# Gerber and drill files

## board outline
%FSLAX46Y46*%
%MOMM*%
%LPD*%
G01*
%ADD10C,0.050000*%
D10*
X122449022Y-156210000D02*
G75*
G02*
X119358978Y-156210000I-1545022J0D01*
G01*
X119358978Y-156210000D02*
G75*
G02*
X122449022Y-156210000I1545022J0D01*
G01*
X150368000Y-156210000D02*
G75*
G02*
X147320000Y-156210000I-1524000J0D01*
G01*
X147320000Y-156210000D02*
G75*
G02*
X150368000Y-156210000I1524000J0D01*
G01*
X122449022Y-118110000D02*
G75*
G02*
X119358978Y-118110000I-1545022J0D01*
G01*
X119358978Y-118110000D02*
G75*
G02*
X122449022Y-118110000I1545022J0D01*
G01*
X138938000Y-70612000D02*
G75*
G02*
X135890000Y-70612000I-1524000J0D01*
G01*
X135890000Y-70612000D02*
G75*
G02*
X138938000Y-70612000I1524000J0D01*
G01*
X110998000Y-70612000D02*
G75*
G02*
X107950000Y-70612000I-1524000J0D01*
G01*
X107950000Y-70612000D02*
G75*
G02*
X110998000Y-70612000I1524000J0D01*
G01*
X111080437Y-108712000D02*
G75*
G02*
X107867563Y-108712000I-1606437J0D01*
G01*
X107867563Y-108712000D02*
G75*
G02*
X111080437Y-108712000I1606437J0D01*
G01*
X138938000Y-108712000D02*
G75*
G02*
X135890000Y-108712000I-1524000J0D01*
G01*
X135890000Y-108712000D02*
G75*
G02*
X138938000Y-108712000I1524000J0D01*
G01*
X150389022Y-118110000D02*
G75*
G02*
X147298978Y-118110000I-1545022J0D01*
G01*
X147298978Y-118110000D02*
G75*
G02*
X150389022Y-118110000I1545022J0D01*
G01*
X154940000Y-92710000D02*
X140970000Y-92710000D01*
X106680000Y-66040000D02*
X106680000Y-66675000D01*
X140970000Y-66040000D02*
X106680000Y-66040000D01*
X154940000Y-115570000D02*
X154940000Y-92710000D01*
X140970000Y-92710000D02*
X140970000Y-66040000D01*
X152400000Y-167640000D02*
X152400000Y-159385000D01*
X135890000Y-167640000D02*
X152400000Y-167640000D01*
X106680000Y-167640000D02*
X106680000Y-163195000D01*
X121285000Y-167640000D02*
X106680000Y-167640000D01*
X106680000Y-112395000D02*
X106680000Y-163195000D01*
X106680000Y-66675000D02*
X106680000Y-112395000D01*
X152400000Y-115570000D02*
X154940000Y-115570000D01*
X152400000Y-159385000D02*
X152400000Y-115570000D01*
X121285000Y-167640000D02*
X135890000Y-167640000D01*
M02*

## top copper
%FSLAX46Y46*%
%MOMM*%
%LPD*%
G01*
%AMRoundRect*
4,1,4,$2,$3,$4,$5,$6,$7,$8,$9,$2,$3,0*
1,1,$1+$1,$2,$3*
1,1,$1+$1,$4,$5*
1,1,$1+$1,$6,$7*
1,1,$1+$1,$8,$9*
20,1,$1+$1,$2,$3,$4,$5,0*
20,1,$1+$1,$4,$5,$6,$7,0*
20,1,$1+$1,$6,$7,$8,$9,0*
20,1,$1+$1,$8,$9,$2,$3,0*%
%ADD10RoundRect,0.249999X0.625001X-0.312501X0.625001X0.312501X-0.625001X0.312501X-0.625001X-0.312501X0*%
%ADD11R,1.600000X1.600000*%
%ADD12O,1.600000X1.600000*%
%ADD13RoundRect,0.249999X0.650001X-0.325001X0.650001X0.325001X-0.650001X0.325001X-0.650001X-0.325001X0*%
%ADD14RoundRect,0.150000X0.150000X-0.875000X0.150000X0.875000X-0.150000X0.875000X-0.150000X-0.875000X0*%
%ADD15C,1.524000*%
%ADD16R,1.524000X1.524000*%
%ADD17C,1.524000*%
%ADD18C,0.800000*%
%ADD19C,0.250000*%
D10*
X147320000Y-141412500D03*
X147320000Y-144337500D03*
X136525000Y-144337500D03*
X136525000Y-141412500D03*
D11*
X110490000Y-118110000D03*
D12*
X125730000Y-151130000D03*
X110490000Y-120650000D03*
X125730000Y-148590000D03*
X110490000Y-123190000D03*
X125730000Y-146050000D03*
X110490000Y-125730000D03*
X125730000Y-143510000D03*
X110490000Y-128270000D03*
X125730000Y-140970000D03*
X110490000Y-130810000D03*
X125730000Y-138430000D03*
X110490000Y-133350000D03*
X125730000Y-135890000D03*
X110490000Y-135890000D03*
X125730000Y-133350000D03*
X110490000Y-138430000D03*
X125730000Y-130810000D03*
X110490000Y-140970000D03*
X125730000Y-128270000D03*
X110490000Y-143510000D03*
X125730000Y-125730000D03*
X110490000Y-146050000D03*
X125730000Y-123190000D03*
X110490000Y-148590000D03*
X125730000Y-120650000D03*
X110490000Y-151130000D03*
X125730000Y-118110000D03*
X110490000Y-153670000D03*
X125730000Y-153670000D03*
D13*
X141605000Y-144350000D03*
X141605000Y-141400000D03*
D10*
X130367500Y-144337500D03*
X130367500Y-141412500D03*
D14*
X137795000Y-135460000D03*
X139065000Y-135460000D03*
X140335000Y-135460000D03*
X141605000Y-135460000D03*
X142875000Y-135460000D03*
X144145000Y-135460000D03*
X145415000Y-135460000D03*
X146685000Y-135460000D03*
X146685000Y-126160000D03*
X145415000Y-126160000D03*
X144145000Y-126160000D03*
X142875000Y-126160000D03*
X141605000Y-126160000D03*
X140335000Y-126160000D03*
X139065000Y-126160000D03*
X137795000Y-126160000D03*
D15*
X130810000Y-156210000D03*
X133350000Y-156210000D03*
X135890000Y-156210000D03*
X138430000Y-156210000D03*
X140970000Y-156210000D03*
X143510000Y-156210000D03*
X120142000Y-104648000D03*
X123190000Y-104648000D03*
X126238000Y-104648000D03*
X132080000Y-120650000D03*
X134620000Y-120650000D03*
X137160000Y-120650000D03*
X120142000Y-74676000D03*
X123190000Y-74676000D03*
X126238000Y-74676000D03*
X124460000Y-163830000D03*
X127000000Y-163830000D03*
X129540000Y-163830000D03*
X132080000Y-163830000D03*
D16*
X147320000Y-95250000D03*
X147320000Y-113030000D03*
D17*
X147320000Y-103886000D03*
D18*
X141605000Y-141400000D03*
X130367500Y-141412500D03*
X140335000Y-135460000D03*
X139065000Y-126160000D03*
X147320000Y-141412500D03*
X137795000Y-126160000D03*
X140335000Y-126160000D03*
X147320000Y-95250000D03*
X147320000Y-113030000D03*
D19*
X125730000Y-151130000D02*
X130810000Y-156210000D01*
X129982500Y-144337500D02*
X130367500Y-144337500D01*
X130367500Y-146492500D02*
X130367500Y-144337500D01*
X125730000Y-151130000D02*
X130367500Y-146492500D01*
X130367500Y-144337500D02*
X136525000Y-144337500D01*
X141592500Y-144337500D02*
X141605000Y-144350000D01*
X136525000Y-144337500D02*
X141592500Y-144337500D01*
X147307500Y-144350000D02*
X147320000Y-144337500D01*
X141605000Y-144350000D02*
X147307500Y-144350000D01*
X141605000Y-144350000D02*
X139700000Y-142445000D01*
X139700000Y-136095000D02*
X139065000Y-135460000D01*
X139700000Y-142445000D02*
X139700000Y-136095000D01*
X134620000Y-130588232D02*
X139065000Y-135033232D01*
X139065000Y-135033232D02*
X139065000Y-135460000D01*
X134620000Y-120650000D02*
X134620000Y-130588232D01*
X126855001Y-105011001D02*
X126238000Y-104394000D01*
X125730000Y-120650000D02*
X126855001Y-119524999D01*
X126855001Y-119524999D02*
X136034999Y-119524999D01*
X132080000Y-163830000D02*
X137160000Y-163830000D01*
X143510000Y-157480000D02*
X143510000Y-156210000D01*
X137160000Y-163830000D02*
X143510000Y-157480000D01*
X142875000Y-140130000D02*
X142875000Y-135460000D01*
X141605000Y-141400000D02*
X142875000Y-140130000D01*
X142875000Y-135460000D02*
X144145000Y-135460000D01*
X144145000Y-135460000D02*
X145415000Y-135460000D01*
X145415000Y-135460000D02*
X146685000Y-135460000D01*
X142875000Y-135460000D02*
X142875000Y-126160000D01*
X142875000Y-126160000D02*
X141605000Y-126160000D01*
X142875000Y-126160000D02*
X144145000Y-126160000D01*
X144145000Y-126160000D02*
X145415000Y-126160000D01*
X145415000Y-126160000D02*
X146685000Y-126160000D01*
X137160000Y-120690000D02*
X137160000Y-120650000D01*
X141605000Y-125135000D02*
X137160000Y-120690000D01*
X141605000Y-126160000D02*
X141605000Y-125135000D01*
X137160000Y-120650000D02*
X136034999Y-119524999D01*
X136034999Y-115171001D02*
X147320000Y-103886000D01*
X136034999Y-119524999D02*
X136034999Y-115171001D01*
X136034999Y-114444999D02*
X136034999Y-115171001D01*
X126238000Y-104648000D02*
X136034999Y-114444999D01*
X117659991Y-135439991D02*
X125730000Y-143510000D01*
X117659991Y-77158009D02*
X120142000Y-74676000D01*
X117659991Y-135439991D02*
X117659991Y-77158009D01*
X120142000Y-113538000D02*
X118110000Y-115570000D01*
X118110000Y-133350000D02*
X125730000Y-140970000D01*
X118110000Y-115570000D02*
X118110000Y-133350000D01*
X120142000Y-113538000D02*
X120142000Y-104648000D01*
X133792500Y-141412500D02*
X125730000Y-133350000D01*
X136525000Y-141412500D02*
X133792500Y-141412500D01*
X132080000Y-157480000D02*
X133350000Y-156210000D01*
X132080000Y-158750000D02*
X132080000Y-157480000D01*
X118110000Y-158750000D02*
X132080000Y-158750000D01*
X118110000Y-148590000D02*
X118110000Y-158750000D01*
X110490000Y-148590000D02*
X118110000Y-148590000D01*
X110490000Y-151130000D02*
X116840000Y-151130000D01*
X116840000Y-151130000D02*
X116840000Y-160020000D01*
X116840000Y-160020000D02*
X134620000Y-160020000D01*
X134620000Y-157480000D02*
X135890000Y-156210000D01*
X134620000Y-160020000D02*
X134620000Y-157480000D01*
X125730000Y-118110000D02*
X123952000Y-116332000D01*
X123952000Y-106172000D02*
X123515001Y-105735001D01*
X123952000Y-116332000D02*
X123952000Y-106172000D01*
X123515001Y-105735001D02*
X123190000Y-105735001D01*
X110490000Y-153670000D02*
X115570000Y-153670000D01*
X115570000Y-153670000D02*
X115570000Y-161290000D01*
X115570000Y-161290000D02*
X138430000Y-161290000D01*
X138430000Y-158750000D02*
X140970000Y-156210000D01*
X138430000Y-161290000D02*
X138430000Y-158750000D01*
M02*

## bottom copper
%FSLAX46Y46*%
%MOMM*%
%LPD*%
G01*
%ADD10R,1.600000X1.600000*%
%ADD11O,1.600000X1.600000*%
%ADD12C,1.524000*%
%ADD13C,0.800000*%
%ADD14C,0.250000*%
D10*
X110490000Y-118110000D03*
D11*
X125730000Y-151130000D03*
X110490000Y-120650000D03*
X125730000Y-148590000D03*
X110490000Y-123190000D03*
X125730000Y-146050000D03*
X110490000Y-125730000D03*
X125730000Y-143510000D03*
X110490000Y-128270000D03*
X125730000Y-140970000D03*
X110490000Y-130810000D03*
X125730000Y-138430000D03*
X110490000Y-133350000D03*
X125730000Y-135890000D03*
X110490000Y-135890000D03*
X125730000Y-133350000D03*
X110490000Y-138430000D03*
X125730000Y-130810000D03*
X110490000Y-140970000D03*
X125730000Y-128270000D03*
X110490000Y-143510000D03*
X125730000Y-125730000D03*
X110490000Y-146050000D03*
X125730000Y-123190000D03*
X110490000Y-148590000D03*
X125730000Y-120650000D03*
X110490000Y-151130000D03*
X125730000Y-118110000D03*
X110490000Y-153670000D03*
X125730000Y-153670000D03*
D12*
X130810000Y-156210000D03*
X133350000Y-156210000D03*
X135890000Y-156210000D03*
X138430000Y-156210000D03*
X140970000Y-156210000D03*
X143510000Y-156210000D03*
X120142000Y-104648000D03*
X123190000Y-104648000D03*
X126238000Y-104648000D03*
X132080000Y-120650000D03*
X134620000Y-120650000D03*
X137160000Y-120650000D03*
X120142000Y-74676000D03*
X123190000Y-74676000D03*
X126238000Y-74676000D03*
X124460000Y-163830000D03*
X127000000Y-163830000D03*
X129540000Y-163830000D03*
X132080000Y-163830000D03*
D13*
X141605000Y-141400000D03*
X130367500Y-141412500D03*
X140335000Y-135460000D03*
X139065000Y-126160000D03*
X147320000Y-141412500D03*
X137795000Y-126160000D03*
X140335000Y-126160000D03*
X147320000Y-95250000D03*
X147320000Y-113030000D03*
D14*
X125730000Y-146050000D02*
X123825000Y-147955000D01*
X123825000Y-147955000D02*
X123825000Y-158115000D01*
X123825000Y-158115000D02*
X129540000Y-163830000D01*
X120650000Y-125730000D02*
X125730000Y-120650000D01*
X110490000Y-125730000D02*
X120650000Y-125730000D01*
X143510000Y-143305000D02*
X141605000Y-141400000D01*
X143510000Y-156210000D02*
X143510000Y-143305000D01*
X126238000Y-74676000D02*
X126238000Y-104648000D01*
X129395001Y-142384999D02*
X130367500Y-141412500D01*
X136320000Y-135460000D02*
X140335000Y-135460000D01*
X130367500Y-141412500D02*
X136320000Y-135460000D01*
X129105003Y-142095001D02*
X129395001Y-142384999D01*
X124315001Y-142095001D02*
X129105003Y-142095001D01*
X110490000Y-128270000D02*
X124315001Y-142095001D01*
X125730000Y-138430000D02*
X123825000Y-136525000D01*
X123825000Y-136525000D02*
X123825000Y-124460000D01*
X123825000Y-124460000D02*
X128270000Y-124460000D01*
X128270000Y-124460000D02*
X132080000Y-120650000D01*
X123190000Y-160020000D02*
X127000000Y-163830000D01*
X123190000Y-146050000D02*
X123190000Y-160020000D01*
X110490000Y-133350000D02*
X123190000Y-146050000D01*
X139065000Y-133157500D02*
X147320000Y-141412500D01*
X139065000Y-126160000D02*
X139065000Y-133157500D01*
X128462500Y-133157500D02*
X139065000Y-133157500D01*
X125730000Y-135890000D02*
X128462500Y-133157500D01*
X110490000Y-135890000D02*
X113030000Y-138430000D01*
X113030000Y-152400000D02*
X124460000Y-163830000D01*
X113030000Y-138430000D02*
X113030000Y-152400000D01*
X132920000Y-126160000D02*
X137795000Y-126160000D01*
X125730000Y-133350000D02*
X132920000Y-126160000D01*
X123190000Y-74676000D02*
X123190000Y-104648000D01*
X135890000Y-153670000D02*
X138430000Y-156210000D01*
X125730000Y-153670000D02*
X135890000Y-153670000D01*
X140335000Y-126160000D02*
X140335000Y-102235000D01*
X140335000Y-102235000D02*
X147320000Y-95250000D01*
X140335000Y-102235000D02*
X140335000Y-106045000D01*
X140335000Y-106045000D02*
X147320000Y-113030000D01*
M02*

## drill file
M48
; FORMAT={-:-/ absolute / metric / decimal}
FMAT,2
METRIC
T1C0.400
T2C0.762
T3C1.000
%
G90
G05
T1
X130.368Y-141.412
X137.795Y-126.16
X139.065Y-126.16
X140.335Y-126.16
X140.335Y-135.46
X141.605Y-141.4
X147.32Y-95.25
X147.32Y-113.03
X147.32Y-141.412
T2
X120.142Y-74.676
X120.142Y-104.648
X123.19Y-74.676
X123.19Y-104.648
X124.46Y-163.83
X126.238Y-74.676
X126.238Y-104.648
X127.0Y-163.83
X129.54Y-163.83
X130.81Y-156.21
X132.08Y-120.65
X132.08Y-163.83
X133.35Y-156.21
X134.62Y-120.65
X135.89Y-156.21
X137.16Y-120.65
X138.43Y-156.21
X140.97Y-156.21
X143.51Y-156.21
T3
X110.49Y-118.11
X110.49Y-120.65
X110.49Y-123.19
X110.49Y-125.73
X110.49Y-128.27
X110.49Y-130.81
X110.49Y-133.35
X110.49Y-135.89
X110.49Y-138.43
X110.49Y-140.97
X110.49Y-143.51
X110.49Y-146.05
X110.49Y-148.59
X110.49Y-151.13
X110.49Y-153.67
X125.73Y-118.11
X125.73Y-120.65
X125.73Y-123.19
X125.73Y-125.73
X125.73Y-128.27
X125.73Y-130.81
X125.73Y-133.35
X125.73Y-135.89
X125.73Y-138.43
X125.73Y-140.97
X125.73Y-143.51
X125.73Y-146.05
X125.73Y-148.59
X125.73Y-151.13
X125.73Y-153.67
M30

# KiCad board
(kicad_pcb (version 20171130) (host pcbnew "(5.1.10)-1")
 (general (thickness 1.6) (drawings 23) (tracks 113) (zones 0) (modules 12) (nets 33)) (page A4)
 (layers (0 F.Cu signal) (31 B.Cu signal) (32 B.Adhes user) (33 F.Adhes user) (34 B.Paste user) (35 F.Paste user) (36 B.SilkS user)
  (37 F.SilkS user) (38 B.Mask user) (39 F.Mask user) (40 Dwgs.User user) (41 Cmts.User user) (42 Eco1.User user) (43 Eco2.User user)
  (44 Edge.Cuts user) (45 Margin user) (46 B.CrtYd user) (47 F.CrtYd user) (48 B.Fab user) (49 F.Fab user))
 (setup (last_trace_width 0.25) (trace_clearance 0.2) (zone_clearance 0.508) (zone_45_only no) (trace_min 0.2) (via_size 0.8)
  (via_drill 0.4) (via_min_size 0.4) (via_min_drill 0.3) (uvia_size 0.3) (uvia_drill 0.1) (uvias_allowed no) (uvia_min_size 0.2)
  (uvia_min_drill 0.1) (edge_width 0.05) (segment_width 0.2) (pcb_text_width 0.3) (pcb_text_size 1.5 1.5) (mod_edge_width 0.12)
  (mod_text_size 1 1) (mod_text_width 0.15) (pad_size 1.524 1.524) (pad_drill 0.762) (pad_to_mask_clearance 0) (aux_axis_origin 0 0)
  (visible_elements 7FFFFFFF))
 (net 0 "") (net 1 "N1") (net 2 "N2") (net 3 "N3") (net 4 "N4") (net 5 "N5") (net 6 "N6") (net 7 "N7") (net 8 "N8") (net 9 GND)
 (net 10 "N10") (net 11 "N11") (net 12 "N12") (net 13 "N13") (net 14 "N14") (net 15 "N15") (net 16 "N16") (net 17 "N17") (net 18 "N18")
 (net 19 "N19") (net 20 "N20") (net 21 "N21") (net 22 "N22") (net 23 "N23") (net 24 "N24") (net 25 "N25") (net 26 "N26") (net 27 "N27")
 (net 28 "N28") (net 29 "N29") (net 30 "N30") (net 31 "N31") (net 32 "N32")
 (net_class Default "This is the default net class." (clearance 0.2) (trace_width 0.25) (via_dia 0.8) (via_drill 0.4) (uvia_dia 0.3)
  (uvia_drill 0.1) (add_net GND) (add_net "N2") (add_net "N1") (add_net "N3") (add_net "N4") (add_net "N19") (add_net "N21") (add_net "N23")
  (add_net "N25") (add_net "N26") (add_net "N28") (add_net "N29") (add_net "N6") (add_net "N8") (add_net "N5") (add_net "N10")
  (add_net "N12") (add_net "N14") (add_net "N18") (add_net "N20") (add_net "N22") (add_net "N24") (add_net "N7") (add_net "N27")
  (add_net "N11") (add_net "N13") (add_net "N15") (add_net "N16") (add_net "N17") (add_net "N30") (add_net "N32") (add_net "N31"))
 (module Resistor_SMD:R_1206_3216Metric (layer F.Cu) (at 147.32 142.875 90)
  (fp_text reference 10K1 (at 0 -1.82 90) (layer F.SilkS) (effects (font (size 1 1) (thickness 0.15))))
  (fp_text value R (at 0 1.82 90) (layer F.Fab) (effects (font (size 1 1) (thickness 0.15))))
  (pad 2 smd roundrect (at 1.4625 0 90) (size 1.125 1.75) (layers F.Cu F.Paste F.Mask) (roundrect_rratio 0.2222213333333333) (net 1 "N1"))
  (pad 1 smd roundrect (at -1.4625 0 90) (size 1.125 1.75) (layers F.Cu F.Paste F.Mask) (roundrect_rratio 0.2222213333333333) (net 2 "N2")))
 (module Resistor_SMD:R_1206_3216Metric (layer F.Cu) (at 136.525 142.875 90)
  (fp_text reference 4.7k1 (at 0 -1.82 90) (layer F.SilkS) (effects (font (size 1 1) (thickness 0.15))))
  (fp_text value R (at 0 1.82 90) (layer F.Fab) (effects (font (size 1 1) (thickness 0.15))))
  (pad 1 smd roundrect (at -1.4625 0 90) (size 1.125 1.75) (layers F.Cu F.Paste F.Mask) (roundrect_rratio 0.2222213333333333) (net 2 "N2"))
  (pad 2 smd roundrect (at 1.4625 0 90) (size 1.125 1.75) (layers F.Cu F.Paste F.Mask) (roundrect_rratio 0.2222213333333333) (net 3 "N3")))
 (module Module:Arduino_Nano (layer F.Cu) (at 110.49 118.11)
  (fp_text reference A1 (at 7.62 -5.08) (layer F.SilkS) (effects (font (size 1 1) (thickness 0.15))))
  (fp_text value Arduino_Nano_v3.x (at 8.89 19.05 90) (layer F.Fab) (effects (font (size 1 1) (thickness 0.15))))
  (pad 1 thru_hole rect (at 0 0) (size 1.6 1.6) (drill 1) (layers *.Cu *.Mask) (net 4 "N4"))
  (pad 17 thru_hole oval (at 15.24 33.02) (size 1.6 1.6) (drill 1) (layers *.Cu *.Mask) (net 2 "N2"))
  (pad 2 thru_hole oval (at 0 2.54) (size 1.6 1.6) (drill 1) (layers *.Cu *.Mask) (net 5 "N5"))
  (pad 18 thru_hole oval (at 15.24 30.48) (size 1.6 1.6) (drill 1) (layers *.Cu *.Mask) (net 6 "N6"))
  (pad 3 thru_hole oval (at 0 5.08) (size 1.6 1.6) (drill 1) (layers *.Cu *.Mask) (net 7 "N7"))
  (pad 19 thru_hole oval (at 15.24 27.94) (size 1.6 1.6) (drill 1) (layers *.Cu *.Mask) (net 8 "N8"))
  (pad 4 thru_hole oval (at 0 7.62) (size 1.6 1.6) (drill 1) (layers *.Cu *.Mask) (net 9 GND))
  (pad 20 thru_hole oval (at 15.24 25.4) (size 1.6 1.6) (drill 1) (layers *.Cu *.Mask) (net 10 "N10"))
  (pad 5 thru_hole oval (at 0 10.16) (size 1.6 1.6) (drill 1) (layers *.Cu *.Mask) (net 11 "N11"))
  (pad 21 thru_hole oval (at 15.24 22.86) (size 1.6 1.6) (drill 1) (layers *.Cu *.Mask) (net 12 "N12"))
  (pad 6 thru_hole oval (at 0 12.7) (size 1.6 1.6) (drill 1) (layers *.Cu *.Mask) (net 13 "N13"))
  (pad 22 thru_hole oval (at 15.24 20.32) (size 1.6 1.6) (drill 1) (layers *.Cu *.Mask) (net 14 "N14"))
  (pad 7 thru_hole oval (at 0 15.24) (size 1.6 1.6) (drill 1) (layers *.Cu *.Mask) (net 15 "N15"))
  (pad 23 thru_hole oval (at 15.24 17.78) (size 1.6 1.6) (drill 1) (layers *.Cu *.Mask) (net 1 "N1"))
  (pad 8 thru_hole oval (at 0 17.78) (size 1.6 1.6) (drill 1) (layers *.Cu *.Mask) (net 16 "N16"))
  (pad 24 thru_hole oval (at 15.24 15.24) (size 1.6 1.6) (drill 1) (layers *.Cu *.Mask) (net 3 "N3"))
  (pad 9 thru_hole oval (at 0 20.32) (size 1.6 1.6) (drill 1) (layers *.Cu *.Mask) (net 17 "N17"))
  (pad 25 thru_hole oval (at 15.24 12.7) (size 1.6 1.6) (drill 1) (layers *.Cu *.Mask) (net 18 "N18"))
  (pad 10 thru_hole oval (at 0 22.86) (size 1.6 1.6) (drill 1) (layers *.Cu *.Mask) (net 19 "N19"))
  (pad 26 thru_hole oval (at 15.24 10.16) (size 1.6 1.6) (drill 1) (layers *.Cu *.Mask) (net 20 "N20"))
  (pad 11 thru_hole oval (at 0 25.4) (size 1.6 1.6) (drill 1) (layers *.Cu *.Mask) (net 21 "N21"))
  (pad 27 thru_hole oval (at 15.24 7.62) (size 1.6 1.6) (drill 1) (layers *.Cu *.Mask) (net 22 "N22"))
  (pad 12 thru_hole oval (at 0 27.94) (size 1.6 1.6) (drill 1) (layers *.Cu *.Mask) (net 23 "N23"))
  (pad 28 thru_hole oval (at 15.24 5.08) (size 1.6 1.6) (drill 1) (layers *.Cu *.Mask) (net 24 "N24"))
  (pad 13 thru_hole oval (at 0 30.48) (size 1.6 1.6) (drill 1) (layers *.Cu *.Mask) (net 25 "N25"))
  (pad 29 thru_hole oval (at 15.24 2.54) (size 1.6 1.6) (drill 1) (layers *.Cu *.Mask) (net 9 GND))
  (pad 14 thru_hole oval (at 0 33.02) (size 1.6 1.6) (drill 1) (layers *.Cu *.Mask) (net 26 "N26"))
  (pad 30 thru_hole oval (at 15.24 0) (size 1.6 1.6) (drill 1) (layers *.Cu *.Mask) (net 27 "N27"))
  (pad 15 thru_hole oval (at 0 35.56) (size 1.6 1.6) (drill 1) (layers *.Cu *.Mask) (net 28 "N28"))
  (pad 16 thru_hole oval (at 15.24 35.56) (size 1.6 1.6) (drill 1) (layers *.Cu *.Mask) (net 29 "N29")))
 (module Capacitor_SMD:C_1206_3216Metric (layer F.Cu) (at 141.605 142.875 90)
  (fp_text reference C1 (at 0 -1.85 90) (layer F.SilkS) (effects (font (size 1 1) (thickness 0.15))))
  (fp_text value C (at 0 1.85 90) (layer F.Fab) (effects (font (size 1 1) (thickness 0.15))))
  (pad 1 smd roundrect (at -1.475 0 90) (size 1.15 1.8) (layers F.Cu F.Paste F.Mask) (roundrect_rratio 0.2173904347826087) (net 2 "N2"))
  (pad 2 smd roundrect (at 1.475 0 90) (size 1.15 1.8) (layers F.Cu F.Paste F.Mask) (roundrect_rratio 0.2173904347826087) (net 9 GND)))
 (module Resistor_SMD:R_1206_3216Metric (layer F.Cu) (at 130.3675 142.875 90)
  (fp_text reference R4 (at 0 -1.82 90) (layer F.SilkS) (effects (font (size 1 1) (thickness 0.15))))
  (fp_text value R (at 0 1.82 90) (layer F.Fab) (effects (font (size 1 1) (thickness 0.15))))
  (pad 1 smd roundrect (at -1.4625 0 90) (size 1.125 1.75) (layers F.Cu F.Paste F.Mask) (roundrect_rratio 0.2222213333333333) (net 2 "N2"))
  (pad 2 smd roundrect (at 1.4625 0 90) (size 1.125 1.75) (layers F.Cu F.Paste F.Mask) (roundrect_rratio 0.2222213333333333) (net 11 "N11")))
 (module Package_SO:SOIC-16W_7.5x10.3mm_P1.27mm (layer F.Cu) (at 142.24 130.81 90)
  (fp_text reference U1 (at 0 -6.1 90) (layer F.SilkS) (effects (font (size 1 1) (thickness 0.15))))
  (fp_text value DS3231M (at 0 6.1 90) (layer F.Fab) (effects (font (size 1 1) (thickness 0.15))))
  (pad 1 smd roundrect (at -4.65 -4.445 90) (size 2.05 0.6) (layers F.Cu F.Paste F.Mask) (roundrect_rratio 0.25) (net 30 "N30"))
  (pad 2 smd roundrect (at -4.65 -3.175 90) (size 2.05 0.6) (layers F.Cu F.Paste F.Mask) (roundrect_rratio 0.25) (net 2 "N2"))
  (pad 3 smd roundrect (at -4.65 -1.905 90) (size 2.05 0.6) (layers F.Cu F.Paste F.Mask) (roundrect_rratio 0.25) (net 11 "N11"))
  (pad 4 smd roundrect (at -4.65 -0.635 90) (size 2.05 0.6) (layers F.Cu F.Paste F.Mask) (roundrect_rratio 0.25) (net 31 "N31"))
  (pad 5 smd roundrect (at -4.65 0.635 90) (size 2.05 0.6) (layers F.Cu F.Paste F.Mask) (roundrect_rratio 0.25) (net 9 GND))
  (pad 6 smd roundrect (at -4.65 1.905 90) (size 2.05 0.6) (layers F.Cu F.Paste F.Mask) (roundrect_rratio 0.25) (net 9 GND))
  (pad 7 smd roundrect (at -4.65 3.175 90) (size 2.05 0.6) (layers F.Cu F.Paste F.Mask) (roundrect_rratio 0.25) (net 9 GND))
  (pad 8 smd roundrect (at -4.65 4.445 90) (size 2.05 0.6) (layers F.Cu F.Paste F.Mask) (roundrect_rratio 0.25) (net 9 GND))
  (pad 9 smd roundrect (at 4.65 4.445 90) (size 2.05 0.6) (layers F.Cu F.Paste F.Mask) (roundrect_rratio 0.25) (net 9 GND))
  (pad 10 smd roundrect (at 4.65 3.175 90) (size 2.05 0.6) (layers F.Cu F.Paste F.Mask) (roundrect_rratio 0.25) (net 9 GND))
  (pad 11 smd roundrect (at 4.65 1.905 90) (size 2.05 0.6) (layers F.Cu F.Paste F.Mask) (roundrect_rratio 0.25) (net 9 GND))
  (pad 12 smd roundrect (at 4.65 0.635 90) (size 2.05 0.6) (layers F.Cu F.Paste F.Mask) (roundrect_rratio 0.25) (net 9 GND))
  (pad 13 smd roundrect (at 4.65 -0.635 90) (size 2.05 0.6) (layers F.Cu F.Paste F.Mask) (roundrect_rratio 0.25) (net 9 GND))
  (pad 14 smd roundrect (at 4.65 -1.905 90) (size 2.05 0.6) (layers F.Cu F.Paste F.Mask) (roundrect_rratio 0.25) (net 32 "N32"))
  (pad 15 smd roundrect (at 4.65 -3.175 90) (size 2.05 0.6) (layers F.Cu F.Paste F.Mask) (roundrect_rratio 0.25) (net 1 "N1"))
  (pad 16 smd roundrect (at 4.65 -4.445 90) (size 2.05 0.6) (layers F.Cu F.Paste F.Mask) (roundrect_rratio 0.25) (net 3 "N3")))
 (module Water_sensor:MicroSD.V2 (layer F.Cu) (at 138.43 153.67)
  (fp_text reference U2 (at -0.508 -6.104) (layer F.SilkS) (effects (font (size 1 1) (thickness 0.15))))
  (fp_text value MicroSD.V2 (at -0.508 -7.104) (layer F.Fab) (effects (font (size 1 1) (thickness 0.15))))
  (pad 1 thru_hole circle (at -7.62 2.54) (size 1.524 1.524) (drill 0.762) (layers *.Cu *.Mask) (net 2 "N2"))
  (pad 2 thru_hole circle (at -5.08 2.54) (size 1.524 1.524) (drill 0.762) (layers *.Cu *.Mask) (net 25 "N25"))
  (pad 3 thru_hole circle (at -2.54 2.54) (size 1.524 1.524) (drill 0.762) (layers *.Cu *.Mask) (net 26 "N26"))
  (pad 4 thru_hole circle (at 0 2.54) (size 1.524 1.524) (drill 0.762) (layers *.Cu *.Mask) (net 29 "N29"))
  (pad 5 thru_hole circle (at 2.54 2.54) (size 1.524 1.524) (drill 0.762) (layers *.Cu *.Mask) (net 28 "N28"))
  (pad 6 thru_hole circle (at 5.08 2.54) (size 1.524 1.524) (drill 0.762) (layers *.Cu *.Mask) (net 9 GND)))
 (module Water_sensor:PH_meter (layer F.Cu) (at 123.19 105.664)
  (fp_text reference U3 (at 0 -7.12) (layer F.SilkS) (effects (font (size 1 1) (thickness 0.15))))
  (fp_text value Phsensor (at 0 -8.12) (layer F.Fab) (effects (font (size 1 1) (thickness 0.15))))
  (pad 1 thru_hole circle (at -3.048 -1.016) (size 1.524 1.524) (drill 0.762) (layers *.Cu *.Mask) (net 12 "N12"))
  (pad 2 thru_hole circle (at 0 -1.016) (size 1.524 1.524) (drill 0.762) (layers *.Cu *.Mask) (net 22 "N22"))
  (pad 3 thru_hole circle (at 3.048 -1.016) (size 1.524 1.524) (drill 0.762) (layers *.Cu *.Mask) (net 9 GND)))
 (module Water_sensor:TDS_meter (layer B.Cu) (at 134.62 123.19)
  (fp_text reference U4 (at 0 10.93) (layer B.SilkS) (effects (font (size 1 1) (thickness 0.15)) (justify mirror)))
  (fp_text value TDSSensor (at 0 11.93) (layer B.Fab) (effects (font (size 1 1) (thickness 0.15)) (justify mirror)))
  (pad 1 thru_hole circle (at -2.54 -2.54) (size 1.524 1.524) (drill 0.762) (layers *.Cu *.Mask) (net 14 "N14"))
  (pad 2 thru_hole circle (at 0 -2.54) (size 1.524 1.524) (drill 0.762) (layers *.Cu *.Mask) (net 2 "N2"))
  (pad 3 thru_hole circle (at 2.54 -2.54) (size 1.524 1.524) (drill 0.762) (layers *.Cu *.Mask) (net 9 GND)))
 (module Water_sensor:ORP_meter (layer B.Cu) (at 123.19 73.66)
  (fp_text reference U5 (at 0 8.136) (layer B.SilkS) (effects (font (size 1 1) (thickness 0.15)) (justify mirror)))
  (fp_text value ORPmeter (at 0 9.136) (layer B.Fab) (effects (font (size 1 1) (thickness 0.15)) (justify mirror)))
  (pad 1 thru_hole circle (at -3.048 1.016) (size 1.524 1.524) (drill 0.762) (layers *.Cu *.Mask F.SilkS) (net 10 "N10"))
  (pad 2 thru_hole circle (at 0 1.016) (size 1.524 1.524) (drill 0.762) (layers *.Cu *.Mask F.SilkS) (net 22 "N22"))
  (pad 3 thru_hole circle (at 3.048 1.016) (size 1.524 1.524) (drill 0.762) (layers *.Cu *.Mask F.SilkS) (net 9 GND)))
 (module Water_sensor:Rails (layer F.Cu) (at 128.27 161.29)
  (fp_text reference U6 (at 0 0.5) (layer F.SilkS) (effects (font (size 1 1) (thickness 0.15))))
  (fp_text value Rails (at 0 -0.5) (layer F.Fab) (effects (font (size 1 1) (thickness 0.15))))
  (pad 1 thru_hole circle (at -3.81 2.54) (size 1.524 1.524) (drill 0.762) (layers *.Cu *.Mask) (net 16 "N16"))
  (pad 2 thru_hole circle (at -1.27 2.54) (size 1.524 1.524) (drill 0.762) (layers *.Cu *.Mask) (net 15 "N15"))
  (pad 3 thru_hole circle (at 1.27 2.54) (size 1.524 1.524) (drill 0.762) (layers *.Cu *.Mask) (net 8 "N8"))
  (pad 4 thru_hole circle (at 3.81 2.54) (size 1.524 1.524) (drill 0.762) (layers *.Cu *.Mask) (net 9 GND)))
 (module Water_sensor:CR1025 (layer F.Cu) (at 147.32 110.49)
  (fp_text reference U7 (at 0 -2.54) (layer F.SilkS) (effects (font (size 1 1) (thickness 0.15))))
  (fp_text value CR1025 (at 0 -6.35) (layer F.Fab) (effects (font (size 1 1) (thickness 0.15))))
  (pad 1 smd rect (at 0 -15.24) (size 1.524 1.524) (layers F.Cu F.Paste F.Mask) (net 32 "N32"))
  (pad 2 smd rect (at 0 2.54) (size 1.524 1.524) (layers F.Cu F.Paste F.Mask) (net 32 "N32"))
  (pad 3 smd circle (at 0 -6.604) (size 1.524 1.524) (layers F.Cu F.Paste F.Mask) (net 9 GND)))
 (gr_circle (center 120.904 156.21) (end 121.158 154.686) (layer Edge.Cuts) (width 0.05))
 (gr_circle (center 148.844 156.21) (end 148.844 157.734) (layer Edge.Cuts) (width 0.05))
 (gr_circle (center 120.904 118.11) (end 120.65 116.586) (layer Edge.Cuts) (width 0.05))
 (gr_circle (center 137.414 70.612) (end 137.414 69.088) (layer Edge.Cuts) (width 0.05))
 (gr_circle (center 109.474 70.612) (end 109.474 69.088) (layer Edge.Cuts) (width 0.05))
 (gr_circle (center 109.474 108.712) (end 109.982 107.188) (layer Edge.Cuts) (width 0.05))
 (gr_circle (center 137.414 108.712) (end 137.414 107.188) (layer Edge.Cuts) (width 0.05))
 (gr_circle (center 148.844 118.11) (end 149.098 116.586) (layer Edge.Cuts) (width 0.05))
 (gr_line (start 154.94 92.71) (end 140.97 92.71) (layer Edge.Cuts) (width 0.05))
 (gr_line (start 106.68 66.04) (end 106.68 66.675) (layer Edge.Cuts) (width 0.05))
 (gr_line (start 140.97 66.04) (end 106.68 66.04) (layer Edge.Cuts) (width 0.05))
 (gr_line (start 154.94 115.57) (end 154.94 92.71) (layer Edge.Cuts) (width 0.05))
 (gr_line (start 140.97 92.71) (end 140.97 66.04) (layer Edge.Cuts) (width 0.05))
 (gr_line (start 152.4 167.64) (end 152.4 159.385) (layer Edge.Cuts) (width 0.05))
 (gr_line (start 135.89 167.64) (end 152.4 167.64) (layer Edge.Cuts) (width 0.05))
 (gr_line (start 106.68 167.64) (end 106.68 163.195) (layer Edge.Cuts) (width 0.05))
 (gr_line (start 121.285 167.64) (end 106.68 167.64) (layer Edge.Cuts) (width 0.05))
 (gr_line (start 106.68 112.395) (end 106.68 163.195) (layer Edge.Cuts) (width 0.05))
 (gr_line (start 106.68 66.675) (end 106.68 112.395) (layer Edge.Cuts) (width 0.05))
 (gr_line (start 152.4 115.57) (end 154.94 115.57) (layer Edge.Cuts) (width 0.05))
 (gr_line (start 152.4 159.385) (end 152.4 115.57) (layer Edge.Cuts) (width 0.05))
 (gr_line (start 121.285 167.64) (end 135.89 167.64) (layer Edge.Cuts) (width 0.05))
 (segment (start 125.73 151.13) (end 130.81 156.21) (width 0.25) (layer F.Cu) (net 2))
 (segment (start 129.9825 144.3375) (end 130.3675 144.3375) (width 0.25) (layer F.Cu) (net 2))
 (segment (start 130.3675 146.4925) (end 130.3675 144.3375) (width 0.25) (layer F.Cu) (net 2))
 (segment (start 125.73 151.13) (end 130.3675 146.4925) (width 0.25) (layer F.Cu) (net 2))
 (segment (start 130.3675 144.3375) (end 136.525 144.3375) (width 0.25) (layer F.Cu) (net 2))
 (segment (start 141.5925 144.3375) (end 141.605 144.35) (width 0.25) (layer F.Cu) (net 2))
 (segment (start 136.525 144.3375) (end 141.5925 144.3375) (width 0.25) (layer F.Cu) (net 2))
 (segment (start 147.3075 144.35) (end 147.32 144.3375) (width 0.25) (layer F.Cu) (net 2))
 (segment (start 141.605 144.35) (end 147.3075 144.35) (width 0.25) (layer F.Cu) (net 2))
 (segment (start 141.605 144.35) (end 139.7 142.445) (width 0.25) (layer F.Cu) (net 2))
 (segment (start 139.7 136.095) (end 139.065 135.46) (width 0.25) (layer F.Cu) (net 2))
 (segment (start 139.7 142.445) (end 139.7 136.095) (width 0.25) (layer F.Cu) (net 2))
 (segment (start 134.62 130.588232) (end 139.065 135.033232) (width 0.25) (layer F.Cu) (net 2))
 (segment (start 139.065 135.033232) (end 139.065 135.46) (width 0.25) (layer F.Cu) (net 2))
 (segment (start 134.62 120.65) (end 134.62 130.588232) (width 0.25) (layer F.Cu) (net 2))
 (segment (start 125.73 146.05) (end 123.825 147.955) (width 0.25) (layer B.Cu) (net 8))
 (segment (start 123.825 147.955) (end 123.825 158.115) (width 0.25) (layer B.Cu) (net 8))
 (segment (start 123.825 158.115) (end 129.54 163.83) (width 0.25) (layer B.Cu) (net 8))
 (segment (start 126.855001 105.011001) (end 126.238 104.394) (width 0.25) (layer F.Cu) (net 9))
 (segment (start 125.73 120.65) (end 126.855001 119.524999) (width 0.25) (layer F.Cu) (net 9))
 (segment (start 126.855001 119.524999) (end 136.034999 119.524999) (width 0.25) (layer F.Cu) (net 9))
 (segment (start 120.65 125.73) (end 125.73 120.65) (width 0.25) (layer B.Cu) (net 9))
 (segment (start 110.49 125.73) (end 120.65 125.73) (width 0.25) (layer B.Cu) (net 9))
 (segment (start 132.08 163.83) (end 137.16 163.83) (width 0.25) (layer F.Cu) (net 9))
 (segment (start 143.51 157.48) (end 143.51 156.21) (width 0.25) (layer F.Cu) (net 9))
 (segment (start 137.16 163.83) (end 143.51 157.48) (width 0.25) (layer F.Cu) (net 9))
 (via (at 141.605 141.4) (size 0.8) (drill 0.4) (layers F.Cu B.Cu) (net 9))
 (segment (start 143.51 143.305) (end 141.605 141.4) (width 0.25) (layer B.Cu) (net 9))
 (segment (start 143.51 156.21) (end 143.51 143.305) (width 0.25) (layer B.Cu) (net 9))
 (segment (start 142.875 140.13) (end 142.875 135.46) (width 0.25) (layer F.Cu) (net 9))
 (segment (start 141.605 141.4) (end 142.875 140.13) (width 0.25) (layer F.Cu) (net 9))
 (segment (start 142.875 135.46) (end 144.145 135.46) (width 0.25) (layer F.Cu) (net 9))
 (segment (start 144.145 135.46) (end 145.415 135.46) (width 0.25) (layer F.Cu) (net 9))
 (segment (start 145.415 135.46) (end 146.685 135.46) (width 0.25) (layer F.Cu) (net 9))
 (segment (start 142.875 135.46) (end 142.875 126.16) (width 0.25) (layer F.Cu) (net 9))
 (segment (start 142.875 126.16) (end 141.605 126.16) (width 0.25) (layer F.Cu) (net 9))
 (segment (start 142.875 126.16) (end 144.145 126.16) (width 0.25) (layer F.Cu) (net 9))
 (segment (start 144.145 126.16) (end 145.415 126.16) (width 0.25) (layer F.Cu) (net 9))
 (segment (start 145.415 126.16) (end 146.685 126.16) (width 0.25) (layer F.Cu) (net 9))
 (segment (start 137.16 120.69) (end 137.16 120.65) (width 0.25) (layer F.Cu) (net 9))
 (segment (start 141.605 125.135) (end 137.16 120.69) (width 0.25) (layer F.Cu) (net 9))
 (segment (start 141.605 126.16) (end 141.605 125.135) (width 0.25) (layer F.Cu) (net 9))
 (segment (start 137.16 120.65) (end 136.034999 119.524999) (width 0.25) (layer F.Cu) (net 9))
 (segment (start 136.034999 115.171001) (end 147.32 103.886) (width 0.25) (layer F.Cu) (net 9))
 (segment (start 136.034999 119.524999) (end 136.034999 115.171001) (width 0.25) (layer F.Cu) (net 9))
 (segment (start 136.034999 114.444999) (end 136.034999 115.171001) (width 0.25) (layer F.Cu) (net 9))
 (segment (start 126.238 104.648) (end 136.034999 114.444999) (width 0.25) (layer F.Cu) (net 9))
 (segment (start 126.238 74.676) (end 126.238 104.648) (width 0.25) (layer B.Cu) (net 9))
 (segment (start 117.659991 135.439991) (end 125.73 143.51) (width 0.25) (layer F.Cu) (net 10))
 (segment (start 117.659991 77.158009) (end 120.142 74.676) (width 0.25) (layer F.Cu) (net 10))
 (segment (start 117.659991 135.439991) (end 117.659991 77.158009) (width 0.25) (layer F.Cu) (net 10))
 (via (at 130.3675 141.4125) (size 0.8) (drill 0.4) (layers F.Cu B.Cu) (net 11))
 (segment (start 129.395001 142.384999) (end 130.3675 141.4125) (width 0.25) (layer B.Cu) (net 11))
 (via (at 140.335 135.46) (size 0.8) (drill 0.4) (layers F.Cu B.Cu) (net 11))
 (segment (start 136.32 135.46) (end 140.335 135.46) (width 0.25) (layer B.Cu) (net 11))
 (segment (start 130.3675 141.4125) (end 136.32 135.46) (width 0.25) (layer B.Cu) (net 11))
 (segment (start 129.105003 142.095001) (end 129.395001 142.384999) (width 0.25) (layer B.Cu) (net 11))
 (segment (start 124.315001 142.095001) (end 129.105003 142.095001) (width 0.25) (layer B.Cu) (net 11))
 (segment (start 110.49 128.27) (end 124.315001 142.095001) (width 0.25) (layer B.Cu) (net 11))
 (segment (start 120.142 113.538) (end 118.11 115.57) (width 0.25) (layer F.Cu) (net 12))
 (segment (start 118.11 133.35) (end 125.73 140.97) (width 0.25) (layer F.Cu) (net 12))
 (segment (start 118.11 115.57) (end 118.11 133.35) (width 0.25) (layer F.Cu) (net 12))
 (segment (start 120.142 113.538) (end 120.142 104.648) (width 0.25) (layer F.Cu) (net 12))
 (segment (start 125.73 138.43) (end 123.825 136.525) (width 0.25) (layer B.Cu) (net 14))
 (segment (start 123.825 136.525) (end 123.825 124.46) (width 0.25) (layer B.Cu) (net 14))
 (segment (start 123.825 124.46) (end 128.27 124.46) (width 0.25) (layer B.Cu) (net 14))
 (segment (start 128.27 124.46) (end 132.08 120.65) (width 0.25) (layer B.Cu) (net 14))
 (segment (start 123.19 160.02) (end 127 163.83) (width 0.25) (layer B.Cu) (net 15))
 (segment (start 123.19 146.05) (end 123.19 160.02) (width 0.25) (layer B.Cu) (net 15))
 (segment (start 110.49 133.35) (end 123.19 146.05) (width 0.25) (layer B.Cu) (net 15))
 (via (at 139.065 126.16) (size 0.8) (drill 0.4) (layers F.Cu B.Cu) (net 1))
 (via (at 147.32 141.4125) (size 0.8) (drill 0.4) (layers F.Cu B.Cu) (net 1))
 (segment (start 139.065 133.1575) (end 147.32 141.4125) (width 0.25) (layer B.Cu) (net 1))
 (segment (start 139.065 126.16) (end 139.065 133.1575) (width 0.25) (layer B.Cu) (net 1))
 (segment (start 128.4625 133.1575) (end 139.065 133.1575) (width 0.25) (layer B.Cu) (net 1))
 (segment (start 125.73 135.89) (end 128.4625 133.1575) (width 0.25) (layer B.Cu) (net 1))
 (segment (start 110.49 135.89) (end 113.03 138.43) (width 0.25) (layer B.Cu) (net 16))
 (segment (start 113.03 152.4) (end 124.46 163.83) (width 0.25) (layer B.Cu) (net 16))
 (segment (start 113.03 138.43) (end 113.03 152.4) (width 0.25) (layer B.Cu) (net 16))
 (segment (start 133.7925 141.4125) (end 125.73 133.35) (width 0.25) (layer F.Cu) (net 3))
 (segment (start 136.525 141.4125) (end 133.7925 141.4125) (width 0.25) (layer F.Cu) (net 3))
 (segment (start 132.92 126.16) (end 137.795 126.16) (width 0.25) (layer B.Cu) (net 3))
 (segment (start 125.73 133.35) (end 132.92 126.16) (width 0.25) (layer B.Cu) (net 3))
 (via (at 137.795 126.16) (size 0.8) (drill 0.4) (layers F.Cu B.Cu) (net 3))
 (segment (start 123.19 74.676) (end 123.19 104.648) (width 0.25) (layer B.Cu) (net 22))
 (segment (start 132.08 157.48) (end 133.35 156.21) (width 0.25) (layer F.Cu) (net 25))
 (segment (start 132.08 158.75) (end 132.08 157.48) (width 0.25) (layer F.Cu) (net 25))
 (segment (start 118.11 158.75) (end 132.08 158.75) (width 0.25) (layer F.Cu) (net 25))
 (segment (start 118.11 148.59) (end 118.11 158.75) (width 0.25) (layer F.Cu) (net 25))
 (segment (start 110.49 148.59) (end 118.11 148.59) (width 0.25) (layer F.Cu) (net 25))
 (segment (start 110.49 151.13) (end 116.84 151.13) (width 0.25) (layer F.Cu) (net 26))
 (segment (start 116.84 151.13) (end 116.84 160.02) (width 0.25) (layer F.Cu) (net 26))
 (segment (start 116.84 160.02) (end 134.62 160.02) (width 0.25) (layer F.Cu) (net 26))
 (segment (start 134.62 157.48) (end 135.89 156.21) (width 0.25) (layer F.Cu) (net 26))
 (segment (start 134.62 160.02) (end 134.62 157.48) (width 0.25) (layer F.Cu) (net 26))
 (segment (start 125.73 118.11) (end 123.952 116.332) (width 0.25) (layer F.Cu) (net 27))
 (segment (start 123.952 106.172) (end 123.515001 105.735001) (width 0.25) (layer F.Cu) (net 27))
 (segment (start 123.952 116.332) (end 123.952 106.172) (width 0.25) (layer F.Cu) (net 27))
 (segment (start 123.515001 105.735001) (end 123.19 105.735001) (width 0.25) (layer F.Cu) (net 27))
 (segment (start 110.49 153.67) (end 115.57 153.67) (width 0.25) (layer F.Cu) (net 28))
 (segment (start 115.57 153.67) (end 115.57 161.29) (width 0.25) (layer F.Cu) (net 28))
 (segment (start 115.57 161.29) (end 138.43 161.29) (width 0.25) (layer F.Cu) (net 28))
 (segment (start 138.43 158.75) (end 140.97 156.21) (width 0.25) (layer F.Cu) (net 28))
 (segment (start 138.43 161.29) (end 138.43 158.75) (width 0.25) (layer F.Cu) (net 28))
 (segment (start 135.89 153.67) (end 138.43 156.21) (width 0.25) (layer B.Cu) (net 29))
 (segment (start 125.73 153.67) (end 135.89 153.67) (width 0.25) (layer B.Cu) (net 29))
 (via (at 140.335 126.16) (size 0.8) (drill 0.4) (layers F.Cu B.Cu) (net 32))
 (segment (start 140.335 126.16) (end 140.335 102.235) (width 0.25) (layer B.Cu) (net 32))
 (via (at 147.32 95.25) (size 0.8) (drill 0.4) (layers F.Cu B.Cu) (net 32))
 (segment (start 140.335 102.235) (end 147.32 95.25) (width 0.25) (layer B.Cu) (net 32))
 (segment (start 140.335 102.235) (end 140.335 106.045) (width 0.25) (layer B.Cu) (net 32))
 (via (at 147.32 113.03) (size 0.8) (drill 0.4) (layers F.Cu B.Cu) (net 32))
 (segment (start 140.335 106.045) (end 147.32 113.03) (width 0.25) (layer B.Cu) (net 32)))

